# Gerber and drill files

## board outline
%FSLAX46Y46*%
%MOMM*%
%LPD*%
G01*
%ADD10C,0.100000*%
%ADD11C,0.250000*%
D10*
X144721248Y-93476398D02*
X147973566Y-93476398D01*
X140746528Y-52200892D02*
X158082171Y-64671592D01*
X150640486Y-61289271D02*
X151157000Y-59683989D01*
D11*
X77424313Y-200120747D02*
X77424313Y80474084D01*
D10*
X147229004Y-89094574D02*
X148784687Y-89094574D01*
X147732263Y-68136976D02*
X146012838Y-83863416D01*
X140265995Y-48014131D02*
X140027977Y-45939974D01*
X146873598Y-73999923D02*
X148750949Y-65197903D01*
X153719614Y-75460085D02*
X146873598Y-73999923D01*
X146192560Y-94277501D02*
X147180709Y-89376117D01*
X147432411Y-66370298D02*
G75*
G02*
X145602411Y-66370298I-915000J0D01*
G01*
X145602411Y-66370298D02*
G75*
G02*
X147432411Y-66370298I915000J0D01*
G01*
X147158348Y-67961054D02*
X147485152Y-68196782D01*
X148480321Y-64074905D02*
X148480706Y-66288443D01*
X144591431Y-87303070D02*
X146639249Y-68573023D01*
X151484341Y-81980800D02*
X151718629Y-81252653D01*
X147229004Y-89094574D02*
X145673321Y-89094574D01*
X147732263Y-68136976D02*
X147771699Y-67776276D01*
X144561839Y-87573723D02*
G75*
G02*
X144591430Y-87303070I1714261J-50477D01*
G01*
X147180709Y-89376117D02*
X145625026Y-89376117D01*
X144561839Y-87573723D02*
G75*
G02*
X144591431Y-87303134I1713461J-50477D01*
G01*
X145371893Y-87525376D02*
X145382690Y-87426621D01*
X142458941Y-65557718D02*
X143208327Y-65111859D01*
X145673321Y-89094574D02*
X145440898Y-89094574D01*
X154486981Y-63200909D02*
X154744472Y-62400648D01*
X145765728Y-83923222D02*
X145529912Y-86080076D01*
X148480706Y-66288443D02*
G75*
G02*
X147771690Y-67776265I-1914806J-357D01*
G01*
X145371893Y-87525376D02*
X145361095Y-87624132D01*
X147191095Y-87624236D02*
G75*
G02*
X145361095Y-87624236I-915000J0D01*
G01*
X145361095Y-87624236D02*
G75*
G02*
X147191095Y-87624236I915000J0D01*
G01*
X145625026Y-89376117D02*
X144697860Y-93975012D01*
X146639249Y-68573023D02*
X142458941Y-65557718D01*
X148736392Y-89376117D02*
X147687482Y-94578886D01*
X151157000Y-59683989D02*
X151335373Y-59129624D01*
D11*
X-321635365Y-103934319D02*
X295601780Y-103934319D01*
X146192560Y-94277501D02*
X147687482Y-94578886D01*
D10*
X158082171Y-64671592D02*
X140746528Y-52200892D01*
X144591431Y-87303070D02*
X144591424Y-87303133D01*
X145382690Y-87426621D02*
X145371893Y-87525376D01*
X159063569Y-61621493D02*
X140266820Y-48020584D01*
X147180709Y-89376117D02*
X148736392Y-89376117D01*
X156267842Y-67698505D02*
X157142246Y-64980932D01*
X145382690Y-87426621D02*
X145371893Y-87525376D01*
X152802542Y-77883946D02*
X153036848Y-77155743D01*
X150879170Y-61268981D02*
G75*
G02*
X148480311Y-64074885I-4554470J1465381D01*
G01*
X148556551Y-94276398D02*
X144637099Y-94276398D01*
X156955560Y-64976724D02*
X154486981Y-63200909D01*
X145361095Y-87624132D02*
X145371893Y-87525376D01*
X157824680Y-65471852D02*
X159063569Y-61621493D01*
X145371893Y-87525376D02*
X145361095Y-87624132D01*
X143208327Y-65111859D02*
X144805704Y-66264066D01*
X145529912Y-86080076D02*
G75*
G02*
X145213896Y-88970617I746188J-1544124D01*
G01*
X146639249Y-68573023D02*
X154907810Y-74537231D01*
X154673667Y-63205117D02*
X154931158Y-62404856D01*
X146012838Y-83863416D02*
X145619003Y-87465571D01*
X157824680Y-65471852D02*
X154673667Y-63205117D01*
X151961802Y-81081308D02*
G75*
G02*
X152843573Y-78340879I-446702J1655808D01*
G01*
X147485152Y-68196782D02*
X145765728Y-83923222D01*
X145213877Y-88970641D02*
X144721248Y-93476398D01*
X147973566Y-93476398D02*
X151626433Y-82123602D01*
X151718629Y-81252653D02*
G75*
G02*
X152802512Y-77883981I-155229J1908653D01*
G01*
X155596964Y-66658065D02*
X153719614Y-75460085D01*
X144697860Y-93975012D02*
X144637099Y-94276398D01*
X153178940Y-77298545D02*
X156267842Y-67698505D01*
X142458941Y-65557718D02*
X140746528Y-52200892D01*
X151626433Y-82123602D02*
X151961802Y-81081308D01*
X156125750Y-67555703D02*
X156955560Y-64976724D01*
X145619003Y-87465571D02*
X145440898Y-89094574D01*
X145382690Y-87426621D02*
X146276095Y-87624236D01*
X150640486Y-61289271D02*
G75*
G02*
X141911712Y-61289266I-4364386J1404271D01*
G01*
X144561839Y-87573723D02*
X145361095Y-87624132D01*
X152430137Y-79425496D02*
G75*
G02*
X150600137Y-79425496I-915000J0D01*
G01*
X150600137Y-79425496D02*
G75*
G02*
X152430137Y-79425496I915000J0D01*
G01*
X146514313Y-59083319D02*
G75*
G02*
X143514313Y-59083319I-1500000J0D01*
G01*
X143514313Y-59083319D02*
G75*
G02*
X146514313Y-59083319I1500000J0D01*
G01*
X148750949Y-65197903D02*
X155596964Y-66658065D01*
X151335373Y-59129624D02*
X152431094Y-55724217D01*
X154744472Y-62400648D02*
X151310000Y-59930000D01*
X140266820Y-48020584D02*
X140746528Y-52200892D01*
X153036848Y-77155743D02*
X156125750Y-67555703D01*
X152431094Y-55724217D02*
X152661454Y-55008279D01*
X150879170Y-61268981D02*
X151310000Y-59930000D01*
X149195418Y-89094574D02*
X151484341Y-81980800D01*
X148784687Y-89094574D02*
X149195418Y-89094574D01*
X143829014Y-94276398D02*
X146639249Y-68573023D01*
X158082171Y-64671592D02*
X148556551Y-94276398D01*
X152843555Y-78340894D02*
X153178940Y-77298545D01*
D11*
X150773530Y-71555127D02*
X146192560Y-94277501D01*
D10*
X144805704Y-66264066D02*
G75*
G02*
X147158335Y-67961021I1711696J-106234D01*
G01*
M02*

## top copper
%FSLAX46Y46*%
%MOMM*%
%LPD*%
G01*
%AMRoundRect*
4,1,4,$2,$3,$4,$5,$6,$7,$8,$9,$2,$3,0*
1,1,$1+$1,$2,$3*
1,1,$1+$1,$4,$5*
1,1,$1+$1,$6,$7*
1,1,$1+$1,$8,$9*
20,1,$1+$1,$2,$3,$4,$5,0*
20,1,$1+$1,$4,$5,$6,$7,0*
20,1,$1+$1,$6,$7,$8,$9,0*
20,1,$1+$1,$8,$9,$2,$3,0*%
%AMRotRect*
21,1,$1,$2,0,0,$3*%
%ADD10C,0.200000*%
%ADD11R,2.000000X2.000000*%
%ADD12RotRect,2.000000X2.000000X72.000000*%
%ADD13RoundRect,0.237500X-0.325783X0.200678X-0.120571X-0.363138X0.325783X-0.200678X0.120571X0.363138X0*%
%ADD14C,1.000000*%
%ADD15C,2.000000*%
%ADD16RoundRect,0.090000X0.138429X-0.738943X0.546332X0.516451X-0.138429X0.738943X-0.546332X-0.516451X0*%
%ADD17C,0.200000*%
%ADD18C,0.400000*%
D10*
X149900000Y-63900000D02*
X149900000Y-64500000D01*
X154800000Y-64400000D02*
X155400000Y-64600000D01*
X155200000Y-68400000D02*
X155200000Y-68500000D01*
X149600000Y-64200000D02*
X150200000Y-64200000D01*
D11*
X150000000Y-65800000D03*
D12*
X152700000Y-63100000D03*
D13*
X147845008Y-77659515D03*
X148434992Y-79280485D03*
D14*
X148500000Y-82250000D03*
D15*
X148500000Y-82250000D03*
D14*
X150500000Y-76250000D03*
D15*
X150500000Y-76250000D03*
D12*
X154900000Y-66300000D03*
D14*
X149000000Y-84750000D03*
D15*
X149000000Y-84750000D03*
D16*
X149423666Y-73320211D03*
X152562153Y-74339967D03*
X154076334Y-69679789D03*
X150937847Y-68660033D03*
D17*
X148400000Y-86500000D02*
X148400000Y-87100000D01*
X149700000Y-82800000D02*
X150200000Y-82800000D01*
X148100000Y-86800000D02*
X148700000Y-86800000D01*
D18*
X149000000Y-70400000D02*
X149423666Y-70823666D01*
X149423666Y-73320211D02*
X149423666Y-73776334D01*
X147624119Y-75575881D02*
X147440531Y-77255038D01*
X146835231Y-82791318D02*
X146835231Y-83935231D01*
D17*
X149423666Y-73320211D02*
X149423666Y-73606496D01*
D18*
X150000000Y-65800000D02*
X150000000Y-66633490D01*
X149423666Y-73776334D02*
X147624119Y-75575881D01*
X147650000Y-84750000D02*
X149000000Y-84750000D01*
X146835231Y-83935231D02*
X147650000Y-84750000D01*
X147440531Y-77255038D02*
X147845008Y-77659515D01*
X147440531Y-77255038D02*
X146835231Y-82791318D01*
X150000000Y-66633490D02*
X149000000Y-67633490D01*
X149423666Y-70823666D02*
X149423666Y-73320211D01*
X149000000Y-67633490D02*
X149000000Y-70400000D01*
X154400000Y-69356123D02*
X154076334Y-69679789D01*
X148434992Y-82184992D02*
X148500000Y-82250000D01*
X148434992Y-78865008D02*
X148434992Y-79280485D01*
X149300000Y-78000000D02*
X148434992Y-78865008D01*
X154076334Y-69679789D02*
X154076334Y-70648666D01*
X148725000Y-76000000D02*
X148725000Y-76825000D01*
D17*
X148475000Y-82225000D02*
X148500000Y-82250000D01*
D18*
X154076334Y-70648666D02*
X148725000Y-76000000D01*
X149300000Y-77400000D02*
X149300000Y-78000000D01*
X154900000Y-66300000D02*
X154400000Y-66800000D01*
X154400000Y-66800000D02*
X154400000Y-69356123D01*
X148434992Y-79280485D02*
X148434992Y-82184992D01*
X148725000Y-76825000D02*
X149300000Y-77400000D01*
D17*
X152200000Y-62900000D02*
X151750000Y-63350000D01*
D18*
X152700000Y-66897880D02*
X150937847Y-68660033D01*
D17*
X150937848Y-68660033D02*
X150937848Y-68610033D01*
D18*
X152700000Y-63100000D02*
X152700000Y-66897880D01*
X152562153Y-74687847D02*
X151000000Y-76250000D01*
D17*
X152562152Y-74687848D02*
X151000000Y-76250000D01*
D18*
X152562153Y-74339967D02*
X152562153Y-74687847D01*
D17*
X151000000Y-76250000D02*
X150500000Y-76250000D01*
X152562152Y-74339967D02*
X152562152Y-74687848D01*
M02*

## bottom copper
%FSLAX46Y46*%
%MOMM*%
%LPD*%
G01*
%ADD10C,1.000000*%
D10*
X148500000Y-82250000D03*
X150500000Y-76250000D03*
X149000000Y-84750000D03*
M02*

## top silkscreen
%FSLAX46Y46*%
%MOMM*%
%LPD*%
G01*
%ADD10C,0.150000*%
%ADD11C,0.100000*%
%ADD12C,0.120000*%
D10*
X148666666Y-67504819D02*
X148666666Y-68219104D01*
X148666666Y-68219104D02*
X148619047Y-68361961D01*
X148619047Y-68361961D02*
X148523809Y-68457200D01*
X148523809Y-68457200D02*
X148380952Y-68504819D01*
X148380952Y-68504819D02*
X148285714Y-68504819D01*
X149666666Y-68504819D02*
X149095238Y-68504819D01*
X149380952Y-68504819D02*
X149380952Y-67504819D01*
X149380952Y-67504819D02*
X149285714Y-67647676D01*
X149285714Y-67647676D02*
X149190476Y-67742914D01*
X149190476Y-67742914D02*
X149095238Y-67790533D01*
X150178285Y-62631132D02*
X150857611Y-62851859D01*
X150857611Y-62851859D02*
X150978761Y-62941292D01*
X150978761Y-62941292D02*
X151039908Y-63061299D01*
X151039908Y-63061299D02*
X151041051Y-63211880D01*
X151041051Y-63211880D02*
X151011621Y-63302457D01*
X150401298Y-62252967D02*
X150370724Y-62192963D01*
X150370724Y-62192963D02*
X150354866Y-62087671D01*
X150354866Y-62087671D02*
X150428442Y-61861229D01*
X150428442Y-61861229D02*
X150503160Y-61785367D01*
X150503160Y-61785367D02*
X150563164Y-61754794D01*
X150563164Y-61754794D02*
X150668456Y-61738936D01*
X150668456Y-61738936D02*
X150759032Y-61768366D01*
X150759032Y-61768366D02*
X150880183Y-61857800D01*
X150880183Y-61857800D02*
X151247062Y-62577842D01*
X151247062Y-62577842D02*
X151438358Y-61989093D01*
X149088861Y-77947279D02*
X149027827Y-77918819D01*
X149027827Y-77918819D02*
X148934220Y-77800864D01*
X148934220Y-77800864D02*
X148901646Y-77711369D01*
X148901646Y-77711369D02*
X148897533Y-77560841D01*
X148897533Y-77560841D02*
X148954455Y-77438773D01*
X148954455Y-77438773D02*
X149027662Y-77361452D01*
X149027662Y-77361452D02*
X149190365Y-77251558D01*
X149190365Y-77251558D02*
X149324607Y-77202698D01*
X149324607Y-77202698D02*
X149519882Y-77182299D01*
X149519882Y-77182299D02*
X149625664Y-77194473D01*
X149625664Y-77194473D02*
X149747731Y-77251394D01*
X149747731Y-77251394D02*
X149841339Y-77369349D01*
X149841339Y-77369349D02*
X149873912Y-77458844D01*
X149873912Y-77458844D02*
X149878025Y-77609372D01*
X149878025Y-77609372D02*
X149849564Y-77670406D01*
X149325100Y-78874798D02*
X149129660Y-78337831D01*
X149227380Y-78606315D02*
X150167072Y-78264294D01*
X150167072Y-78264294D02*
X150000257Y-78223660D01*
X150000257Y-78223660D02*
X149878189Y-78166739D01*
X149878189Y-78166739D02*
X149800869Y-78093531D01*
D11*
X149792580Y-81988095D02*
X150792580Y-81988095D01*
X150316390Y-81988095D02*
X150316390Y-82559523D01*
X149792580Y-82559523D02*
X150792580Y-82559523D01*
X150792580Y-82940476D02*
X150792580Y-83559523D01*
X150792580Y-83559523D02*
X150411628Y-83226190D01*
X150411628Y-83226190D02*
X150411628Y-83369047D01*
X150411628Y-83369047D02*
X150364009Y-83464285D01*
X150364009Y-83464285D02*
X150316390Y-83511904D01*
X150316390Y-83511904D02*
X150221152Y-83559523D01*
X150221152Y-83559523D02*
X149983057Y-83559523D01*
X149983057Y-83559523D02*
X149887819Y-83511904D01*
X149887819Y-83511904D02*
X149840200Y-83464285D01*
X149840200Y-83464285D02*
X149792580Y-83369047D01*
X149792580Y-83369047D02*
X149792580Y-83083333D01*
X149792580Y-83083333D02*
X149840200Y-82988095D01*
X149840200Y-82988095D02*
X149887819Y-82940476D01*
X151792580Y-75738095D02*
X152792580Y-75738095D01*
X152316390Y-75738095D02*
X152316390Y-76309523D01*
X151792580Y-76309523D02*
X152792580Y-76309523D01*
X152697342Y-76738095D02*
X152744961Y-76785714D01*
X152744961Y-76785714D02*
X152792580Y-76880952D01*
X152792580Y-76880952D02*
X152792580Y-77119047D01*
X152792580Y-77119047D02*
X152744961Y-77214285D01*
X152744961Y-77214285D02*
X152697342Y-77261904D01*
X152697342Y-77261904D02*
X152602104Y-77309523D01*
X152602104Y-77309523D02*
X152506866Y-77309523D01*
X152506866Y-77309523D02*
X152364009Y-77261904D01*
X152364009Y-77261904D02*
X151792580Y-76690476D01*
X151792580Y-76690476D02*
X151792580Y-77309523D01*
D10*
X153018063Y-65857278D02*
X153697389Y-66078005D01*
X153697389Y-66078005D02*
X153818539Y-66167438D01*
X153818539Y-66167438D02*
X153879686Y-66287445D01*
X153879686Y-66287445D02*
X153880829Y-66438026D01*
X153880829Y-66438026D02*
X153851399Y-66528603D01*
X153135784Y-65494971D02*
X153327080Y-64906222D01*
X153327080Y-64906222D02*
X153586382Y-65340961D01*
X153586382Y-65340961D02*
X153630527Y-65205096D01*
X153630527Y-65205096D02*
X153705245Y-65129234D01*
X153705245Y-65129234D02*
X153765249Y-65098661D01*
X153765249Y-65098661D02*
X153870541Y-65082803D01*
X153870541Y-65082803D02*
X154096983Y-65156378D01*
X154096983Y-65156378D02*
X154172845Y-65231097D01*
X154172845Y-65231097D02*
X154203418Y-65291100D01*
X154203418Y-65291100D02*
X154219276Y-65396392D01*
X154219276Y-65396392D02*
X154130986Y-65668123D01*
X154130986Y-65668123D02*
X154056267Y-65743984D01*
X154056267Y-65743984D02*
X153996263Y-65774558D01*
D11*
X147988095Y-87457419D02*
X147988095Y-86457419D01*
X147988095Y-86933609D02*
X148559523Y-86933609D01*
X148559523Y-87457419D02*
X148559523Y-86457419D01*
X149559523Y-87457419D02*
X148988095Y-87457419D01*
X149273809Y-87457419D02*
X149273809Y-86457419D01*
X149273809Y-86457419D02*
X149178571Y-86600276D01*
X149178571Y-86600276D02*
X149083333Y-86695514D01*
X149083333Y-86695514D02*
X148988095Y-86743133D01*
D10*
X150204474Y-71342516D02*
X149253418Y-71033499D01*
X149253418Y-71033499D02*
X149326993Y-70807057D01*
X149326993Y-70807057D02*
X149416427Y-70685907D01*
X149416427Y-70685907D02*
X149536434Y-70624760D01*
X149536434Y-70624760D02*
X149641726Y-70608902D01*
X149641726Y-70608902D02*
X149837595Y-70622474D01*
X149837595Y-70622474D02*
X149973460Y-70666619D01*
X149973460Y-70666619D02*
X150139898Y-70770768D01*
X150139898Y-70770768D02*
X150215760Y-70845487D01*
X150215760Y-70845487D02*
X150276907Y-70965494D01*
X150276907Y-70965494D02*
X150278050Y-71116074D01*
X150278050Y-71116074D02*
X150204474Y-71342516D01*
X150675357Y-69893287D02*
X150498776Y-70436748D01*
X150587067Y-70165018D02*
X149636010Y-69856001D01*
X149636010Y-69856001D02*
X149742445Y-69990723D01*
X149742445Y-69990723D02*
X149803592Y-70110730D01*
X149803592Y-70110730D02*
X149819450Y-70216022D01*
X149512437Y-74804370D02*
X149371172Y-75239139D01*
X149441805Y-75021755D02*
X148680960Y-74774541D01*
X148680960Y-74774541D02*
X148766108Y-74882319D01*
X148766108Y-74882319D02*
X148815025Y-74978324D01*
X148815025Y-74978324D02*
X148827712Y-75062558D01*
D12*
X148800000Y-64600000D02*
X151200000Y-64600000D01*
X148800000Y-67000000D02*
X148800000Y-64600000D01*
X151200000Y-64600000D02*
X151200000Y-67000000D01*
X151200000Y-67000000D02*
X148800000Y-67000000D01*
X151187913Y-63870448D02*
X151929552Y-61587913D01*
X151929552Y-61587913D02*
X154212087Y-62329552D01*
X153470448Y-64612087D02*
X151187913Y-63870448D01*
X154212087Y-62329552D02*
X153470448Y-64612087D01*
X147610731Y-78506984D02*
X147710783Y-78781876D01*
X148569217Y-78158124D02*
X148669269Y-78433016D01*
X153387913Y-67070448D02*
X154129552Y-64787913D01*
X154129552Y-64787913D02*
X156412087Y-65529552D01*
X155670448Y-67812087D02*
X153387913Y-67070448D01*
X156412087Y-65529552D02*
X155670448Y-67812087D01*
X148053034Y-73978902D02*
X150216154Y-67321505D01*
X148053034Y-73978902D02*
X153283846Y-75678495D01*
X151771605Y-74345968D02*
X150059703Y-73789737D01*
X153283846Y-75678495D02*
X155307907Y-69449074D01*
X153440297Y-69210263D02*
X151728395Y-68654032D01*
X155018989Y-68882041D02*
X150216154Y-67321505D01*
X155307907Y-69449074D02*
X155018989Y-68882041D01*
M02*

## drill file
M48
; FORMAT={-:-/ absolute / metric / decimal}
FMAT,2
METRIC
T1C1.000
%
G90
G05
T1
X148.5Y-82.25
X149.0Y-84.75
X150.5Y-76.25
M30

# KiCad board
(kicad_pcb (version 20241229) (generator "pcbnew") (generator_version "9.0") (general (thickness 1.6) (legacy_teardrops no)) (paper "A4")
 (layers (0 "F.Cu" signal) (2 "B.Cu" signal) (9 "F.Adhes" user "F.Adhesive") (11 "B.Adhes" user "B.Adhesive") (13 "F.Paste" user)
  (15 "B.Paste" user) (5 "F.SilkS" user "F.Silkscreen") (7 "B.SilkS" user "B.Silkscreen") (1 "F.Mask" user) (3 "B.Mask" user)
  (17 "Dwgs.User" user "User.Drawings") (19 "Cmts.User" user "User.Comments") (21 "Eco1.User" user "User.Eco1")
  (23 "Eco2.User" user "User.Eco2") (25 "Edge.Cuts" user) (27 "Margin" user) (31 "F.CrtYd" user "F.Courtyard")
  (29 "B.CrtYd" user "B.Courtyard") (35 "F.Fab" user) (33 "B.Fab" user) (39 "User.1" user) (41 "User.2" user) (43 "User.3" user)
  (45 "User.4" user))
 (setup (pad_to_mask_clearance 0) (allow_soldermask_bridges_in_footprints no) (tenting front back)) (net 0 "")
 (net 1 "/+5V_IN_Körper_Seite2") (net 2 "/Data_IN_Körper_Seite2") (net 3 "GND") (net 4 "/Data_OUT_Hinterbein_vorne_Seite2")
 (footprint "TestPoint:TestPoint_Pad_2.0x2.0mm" (layer "F.Cu") (at 150 65.8)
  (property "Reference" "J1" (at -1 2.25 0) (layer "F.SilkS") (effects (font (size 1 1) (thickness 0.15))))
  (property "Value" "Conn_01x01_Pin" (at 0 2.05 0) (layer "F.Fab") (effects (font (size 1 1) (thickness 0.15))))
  (fp_line (start -1.2 -1.2) (end 1.2 -1.2) (stroke (width 0.12) (type solid)) (layer "F.SilkS"))
  (fp_line (start -1.2 1.2) (end -1.2 -1.2) (stroke (width 0.12) (type solid)) (layer "F.SilkS"))
  (fp_line (start 1.2 -1.2) (end 1.2 1.2) (stroke (width 0.12) (type solid)) (layer "F.SilkS"))
  (fp_line (start 1.2 1.2) (end -1.2 1.2) (stroke (width 0.12) (type solid)) (layer "F.SilkS"))
  (pad "1" smd rect (at 0 0) (size 2 2) (layers "F.Cu" "F.Mask") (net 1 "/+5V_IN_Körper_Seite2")))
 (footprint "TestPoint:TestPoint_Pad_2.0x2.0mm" (layer "F.Cu") (at 152.7 63.1 72)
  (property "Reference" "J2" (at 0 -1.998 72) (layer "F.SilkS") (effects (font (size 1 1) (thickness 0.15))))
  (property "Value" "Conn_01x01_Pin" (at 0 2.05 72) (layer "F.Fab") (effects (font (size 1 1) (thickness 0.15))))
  (fp_line (start -1.2 -1.199999) (end 1.199999 -1.2) (stroke (width 0.12) (type solid)) (layer "F.SilkS"))
  (fp_line (start 1.199999 -1.2) (end 1.2 1.199999) (stroke (width 0.12) (type solid)) (layer "F.SilkS"))
  (fp_line (start -1.199999 1.2) (end -1.2 -1.199999) (stroke (width 0.12) (type solid)) (layer "F.SilkS"))
  (fp_line (start 1.2 1.199999) (end -1.199999 1.2) (stroke (width 0.12) (type solid)) (layer "F.SilkS"))
  (pad "1" smd rect (at 0 0 72) (size 2 2) (layers "F.Cu" "F.Mask") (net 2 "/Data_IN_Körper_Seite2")))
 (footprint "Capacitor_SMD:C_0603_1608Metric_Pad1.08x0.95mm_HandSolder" (layer "F.Cu") (at 148.14 78.47 -70)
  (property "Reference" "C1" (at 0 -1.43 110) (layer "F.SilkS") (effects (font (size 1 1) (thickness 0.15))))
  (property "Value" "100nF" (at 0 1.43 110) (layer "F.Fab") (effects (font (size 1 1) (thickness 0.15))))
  (fp_line (start -0.146267 0.509999) (end 0.146267 0.51) (stroke (width 0.12) (type solid)) (layer "F.SilkS"))
  (fp_line (start -0.146267 -0.51) (end 0.146267 -0.509999) (stroke (width 0.12) (type solid)) (layer "F.SilkS"))
  (pad "1" smd roundrect (at -0.8625 0 290) (size 1.075 0.95) (layers "F.Cu" "F.Mask" "F.Paste") (roundrect_rratio 0.25)
   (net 1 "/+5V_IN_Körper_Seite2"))
  (pad "2" smd roundrect (at 0.8625 0 290) (size 1.075 0.95) (layers "F.Cu" "F.Mask" "F.Paste") (roundrect_rratio 0.25) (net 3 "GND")))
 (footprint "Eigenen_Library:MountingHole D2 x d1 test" (layer "F.Cu") (at 148.5 82.25)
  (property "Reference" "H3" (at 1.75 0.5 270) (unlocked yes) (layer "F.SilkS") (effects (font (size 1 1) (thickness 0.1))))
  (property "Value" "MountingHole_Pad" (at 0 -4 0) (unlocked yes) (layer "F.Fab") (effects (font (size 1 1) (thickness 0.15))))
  (pad "1" thru_hole circle (at 0 0) (size 1 1) (drill 1) (layers "*.Cu" "*.Mask") (remove_unused_layers no) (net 3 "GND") (zone_connect 2))
  (pad "1" connect circle (at 0 0) (size 2 2) (layers "F.Cu" "F.Mask") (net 3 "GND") (zone_connect 2)))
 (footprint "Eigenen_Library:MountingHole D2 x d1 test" (layer "F.Cu") (at 150.5 76.25)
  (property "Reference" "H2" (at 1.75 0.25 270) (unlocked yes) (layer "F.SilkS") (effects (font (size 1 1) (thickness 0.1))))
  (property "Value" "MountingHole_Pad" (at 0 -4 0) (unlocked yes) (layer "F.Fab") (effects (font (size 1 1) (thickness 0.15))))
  (pad "1" thru_hole circle (at 0 0) (size 1 1) (drill 1) (layers "*.Cu" "*.Mask") (remove_unused_layers no)
   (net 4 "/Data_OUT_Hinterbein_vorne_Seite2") (zone_connect 2))
  (pad "1" connect circle (at 0 0) (size 2 2) (layers "F.Cu" "F.Mask") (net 4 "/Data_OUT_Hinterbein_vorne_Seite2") (zone_connect 2)))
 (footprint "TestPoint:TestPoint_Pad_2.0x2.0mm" (layer "F.Cu") (at 154.9 66.3 72)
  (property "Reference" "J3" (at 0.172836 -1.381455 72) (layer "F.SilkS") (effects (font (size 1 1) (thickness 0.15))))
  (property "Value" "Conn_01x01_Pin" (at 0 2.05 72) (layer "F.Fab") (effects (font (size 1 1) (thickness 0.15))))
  (fp_line (start -1.2 -1.199999) (end 1.199999 -1.2) (stroke (width 0.12) (type solid)) (layer "F.SilkS"))
  (fp_line (start 1.199999 -1.2) (end 1.2 1.199999) (stroke (width 0.12) (type solid)) (layer "F.SilkS"))
  (fp_line (start -1.199999 1.2) (end -1.2 -1.199999) (stroke (width 0.12) (type solid)) (layer "F.SilkS"))
  (fp_line (start 1.2 1.199999) (end -1.199999 1.2) (stroke (width 0.12) (type solid)) (layer "F.SilkS"))
  (pad "1" smd rect (at 0 0 72) (size 2 2) (layers "F.Cu" "F.Mask") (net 3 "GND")))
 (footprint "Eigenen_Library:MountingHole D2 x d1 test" (layer "F.Cu") (at 149 84.75)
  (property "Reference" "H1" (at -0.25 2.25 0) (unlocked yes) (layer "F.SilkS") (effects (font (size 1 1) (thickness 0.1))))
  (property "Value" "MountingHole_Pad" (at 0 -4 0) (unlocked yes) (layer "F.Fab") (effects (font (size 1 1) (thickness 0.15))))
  (pad "1" thru_hole circle (at 0 0) (size 1 1) (drill 1) (layers "*.Cu" "*.Mask") (remove_unused_layers no) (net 1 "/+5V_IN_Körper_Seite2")
   (zone_connect 2))
  (pad "1" connect circle (at 0 0) (size 2 2) (layers "F.Cu" "F.Mask") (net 1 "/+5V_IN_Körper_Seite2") (zone_connect 2)))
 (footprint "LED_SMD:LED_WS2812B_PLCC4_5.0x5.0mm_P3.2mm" (layer "F.Cu") (at 151.75 71.5 72)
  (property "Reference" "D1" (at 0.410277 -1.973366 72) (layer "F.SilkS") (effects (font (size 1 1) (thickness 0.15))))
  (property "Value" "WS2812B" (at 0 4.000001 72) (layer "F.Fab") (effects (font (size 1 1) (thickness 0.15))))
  (fp_line (start -3.500001 -2.750001) (end 3.5 -2.75) (stroke (width 0.12) (type solid)) (layer "F.SilkS"))
  (fp_line (start -3.500001 -2.750001) (end -3.5 2.75) (stroke (width 0.12) (type default)) (layer "F.SilkS"))
  (fp_line (start -2.7 0.9) (end -2.7 -0.9) (stroke (width 0.12) (type default)) (layer "F.SilkS"))
  (fp_line (start -3.5 2.75) (end 3.05 2.75) (stroke (width 0.12) (type solid)) (layer "F.SilkS"))
  (fp_line (start 2.7 0.9) (end 2.7 -0.9) (stroke (width 0.12) (type default)) (layer "F.SilkS"))
  (fp_line (start 3.5 2.299999) (end 3.5 -2.75) (stroke (width 0.12) (type default)) (layer "F.SilkS"))
  (fp_line (start 3.05 2.75) (end 3.5 2.299999) (stroke (width 0.12) (type default)) (layer "F.SilkS"))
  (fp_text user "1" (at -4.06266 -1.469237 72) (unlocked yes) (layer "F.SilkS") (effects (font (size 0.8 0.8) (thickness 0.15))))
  (pad "1" smd roundrect (at -2.45 -1.649999 72) (size 1.5 0.9) (layers "F.Cu" "F.Mask" "F.Paste") (roundrect_rratio 0.1)
   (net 1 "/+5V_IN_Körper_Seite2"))
  (pad "2" smd roundrect (at -2.45 1.650001 72) (size 1.5 0.9) (layers "F.Cu" "F.Mask" "F.Paste") (roundrect_rratio 0.1)
   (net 4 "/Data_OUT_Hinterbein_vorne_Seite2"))
  (pad "3" smd roundrect (at 2.45 1.649999 72) (size 1.5 0.9) (layers "F.Cu" "F.Mask" "F.Paste") (roundrect_rratio 0.1) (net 3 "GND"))
  (pad "4" smd roundrect (at 2.45 -1.650001 72) (size 1.5 0.9) (layers "F.Cu" "F.Mask" "F.Paste") (roundrect_rratio 0.1)
   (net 2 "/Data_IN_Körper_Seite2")))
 (gr_line (start 149.9 63.9) (end 149.9 64.5) (stroke (width 0.2) (type default)) (layer "F.Cu"))
 (gr_line (start 154.8 64.4) (end 155.4 64.6) (stroke (width 0.2) (type default)) (layer "F.Cu"))
 (gr_line (start 155.2 68.4) (end 155.2 68.5) (stroke (width 0.2) (type default)) (layer "F.Cu"))
 (gr_line (start 149.6 64.2) (end 150.2 64.2) (stroke (width 0.2) (type default)) (layer "F.Cu"))
 (gr_line (start 144.721248 93.476398) (end 147.973566 93.476398) (stroke (width 0.1) (type default)) (layer "Edge.Cuts"))
 (gr_line (start 140.746528 52.200892) (end 158.082171 64.671592) (stroke (width 0.1) (type default)) (layer "Edge.Cuts"))
 (gr_line (start 150.640486 61.289271) (end 151.157 59.683989) (stroke (width 0.1) (type default)) (layer "Edge.Cuts"))
 (gr_line (start 77.424313 200.120747) (end 77.424313 -80.474084) (stroke (width 0.25) (type default)) (layer "Edge.Cuts"))
 (gr_line (start 147.229004 89.094574) (end 148.784687 89.094574) (stroke (width 0.1) (type default)) (locked yes) (layer "Edge.Cuts"))
 (gr_line (start 147.732263 68.136976) (end 146.012838 83.863416) (stroke (width 0.1) (type default)) (locked yes) (layer "Edge.Cuts"))
 (gr_line (start 140.265995 48.014131) (end 140.027977 45.939974) (stroke (width 0.1) (type default)) (layer "Edge.Cuts"))
 (gr_line (start 146.873598 73.999923) (end 148.750949 65.197903) (stroke (width 0.1) (type default)) (layer "Edge.Cuts"))
 (gr_line (start 153.719614 75.460085) (end 146.873598 73.999923) (stroke (width 0.1) (type default)) (layer "Edge.Cuts"))
 (gr_line (start 146.19256 94.277501) (end 147.180709 89.376117) (stroke (width 0.1) (type default)) (layer "Edge.Cuts"))
 (gr_circle (center 146.517411 66.370298) (end 147.432411 66.370298) (stroke (width 0.1) (type default)) (fill no) (layer "Edge.Cuts"))
 (gr_line (start 147.158348 67.961054) (end 147.485152 68.196782) (stroke (width 0.1) (type default)) (layer "Edge.Cuts"))
 (gr_line (start 148.480321 64.074905) (end 148.480706 66.288443) (stroke (width 0.1) (type default)) (locked yes) (layer "Edge.Cuts"))
 (gr_line (start 144.591431 87.30307) (end 146.639249 68.573023) (stroke (width 0.1) (type default)) (layer "Edge.Cuts"))
 (gr_line (start 151.484341 81.9808) (end 151.718629 81.252653) (stroke (width 0.1) (type default)) (locked yes) (layer "Edge.Cuts"))
 (gr_line (start 147.229004 89.094574) (end 145.673321 89.094574) (stroke (width 0.1) (type default)) (locked yes) (layer "Edge.Cuts"))
 (gr_line (start 147.732263 68.136976) (end 147.771699 67.776276) (stroke (width 0.1) (type default)) (locked yes) (layer "Edge.Cuts"))
 (gr_arc (start 144.561839 87.573723) (mid 144.571252 87.43784) (end 144.591431 87.30307) (stroke (width 0.1) (type default))
  (layer "Edge.Cuts"))
 (gr_line (start 147.180709 89.376117) (end 145.625026 89.376117) (stroke (width 0.1) (type default)) (layer "Edge.Cuts"))
 (gr_arc (start 144.561839 87.573723) (mid 144.571252 87.43784) (end 144.591424 87.303133) (stroke (width 0.1) (type default))
  (layer "Edge.Cuts"))
 (gr_line (start 145.371893 87.525376) (end 145.38269 87.426621) (stroke (width 0.1) (type default)) (layer "Edge.Cuts"))
 (gr_line (start 142.458941 65.557718) (end 143.208327 65.111859) (stroke (width 0.1) (type default)) (layer "Edge.Cuts"))
 (gr_line (start 145.673321 89.094574) (end 145.440898 89.094574) (stroke (width 0.1) (type default)) (locked yes) (layer "Edge.Cuts"))
 (gr_line (start 154.486981 63.200909) (end 154.744472 62.400648) (stroke (width 0.1) (type default)) (locked yes) (layer "Edge.Cuts"))
 (gr_line (start 145.765728 83.923222) (end 145.529912 86.080076) (stroke (width 0.1) (type default)) (layer "Edge.Cuts"))
 (gr_arc (start 148.480706 66.288443) (mid 148.294469 67.112549) (end 147.771699 67.776276) (stroke (width 0.1) (type default)) (locked yes)
  (layer "Edge.Cuts"))
 (gr_line (start 145.371893 87.525376) (end 145.361095 87.624132) (stroke (width 0.1) (type default)) (layer "Edge.Cuts"))
 (gr_circle (center 146.276095 87.624236) (end 147.191095 87.624236) (stroke (width 0.1) (type default)) (fill no) (layer "Edge.Cuts"))
 (gr_line (start 145.625026 89.376117) (end 144.69786 93.975012) (stroke (width 0.1) (type default)) (layer "Edge.Cuts"))
 (gr_line (start 146.639249 68.573023) (end 142.458941 65.557718) (stroke (width 0.1) (type default)) (layer "Edge.Cuts"))
 (gr_line (start 148.736392 89.376117) (end 147.687482 94.578886) (stroke (width 0.1) (type default)) (layer "Edge.Cuts"))
 (gr_line (start 151.157 59.683989) (end 151.335373 59.129624) (stroke (width 0.1) (type default)) (layer "Edge.Cuts"))
 (gr_line (start -321.635365 103.934319) (end 295.60178 103.934319) (stroke (width 0.25) (type default)) (layer "Edge.Cuts"))
 (gr_line (start 146.19256 94.277501) (end 147.687482 94.578886) (stroke (width 0.25) (type default)) (layer "Edge.Cuts"))
 (gr_line (start 158.082171 64.671592) (end 140.746528 52.200892) (stroke (width 0.1) (type default)) (layer "Edge.Cuts"))
 (gr_line (start 144.591431 87.30307) (end 144.591424 87.303133) (stroke (width 0.1) (type default)) (layer "Edge.Cuts"))
 (gr_line (start 145.38269 87.426621) (end 145.371893 87.525376) (stroke (width 0.1) (type default)) (layer "Edge.Cuts"))
 (gr_line (start 159.063569 61.621493) (end 140.26682 48.020584) (stroke (width 0.1) (type default)) (layer "Edge.Cuts"))
 (gr_line (start 147.180709 89.376117) (end 148.736392 89.376117) (stroke (width 0.1) (type default)) (layer "Edge.Cuts"))
 (gr_line (start 156.267842 67.698505) (end 157.142246 64.980932) (stroke (width 0.1) (type default)) (layer "Edge.Cuts"))
 (gr_line (start 145.38269 87.426621) (end 145.371893 87.525376) (stroke (width 0.1) (type default)) (layer "Edge.Cuts"))
 (gr_line (start 152.802542 77.883946) (end 153.036848 77.155743) (stroke (width 0.1) (type default)) (locked yes) (layer "Edge.Cuts"))
 (gr_arc (start 150.87917 61.268981) (mid 149.961258 62.912638) (end 148.480321 64.074905) (stroke (width 0.1) (type default)) (locked yes)
  (layer "Edge.Cuts"))
 (gr_line (start 148.556551 94.276398) (end 144.637099 94.276398) (stroke (width 0.1) (type default)) (layer "Edge.Cuts"))
 (gr_line (start 156.95556 64.976724) (end 154.486981 63.200909) (stroke (width 0.1) (type default)) (locked yes) (layer "Edge.Cuts"))
 (gr_line (start 145.361095 87.624132) (end 145.371893 87.525376) (stroke (width 0.1) (type default)) (layer "Edge.Cuts"))
 (gr_line (start 157.82468 65.471852) (end 159.063569 61.621493) (stroke (width 0.1) (type default)) (layer "Edge.Cuts"))
 (gr_line (start 145.371893 87.525376) (end 145.361095 87.624132) (stroke (width 0.1) (type default)) (layer "Edge.Cuts"))
 (gr_line (start 143.208327 65.111859) (end 144.805704 66.264066) (stroke (width 0.1) (type default)) (layer "Edge.Cuts"))
 (gr_arc (start 145.529912 86.080076) (mid 147.980947 87.810604) (end 145.213877 88.970641) (stroke (width 0.1) (type default))
  (layer "Edge.Cuts"))
 (gr_line (start 146.639249 68.573023) (end 154.90781 74.537231) (stroke (width 0.1) (type default)) (layer "Edge.Cuts"))
 (gr_line (start 154.673667 63.205117) (end 154.931158 62.404856) (stroke (width 0.1) (type default)) (layer "Edge.Cuts"))
 (gr_line (start 146.012838 83.863416) (end 145.619003 87.465571) (stroke (width 0.1) (type default)) (locked yes) (layer "Edge.Cuts"))
 (gr_line (start 157.82468 65.471852) (end 154.673667 63.205117) (stroke (width 0.1) (type default)) (layer "Edge.Cuts"))
 (gr_arc (start 151.961802 81.081308) (mid 149.882552 78.900244) (end 152.843555 78.340894) (stroke (width 0.1) (type default))
  (layer "Edge.Cuts"))
 (gr_line (start 147.485152 68.196782) (end 145.765728 83.923222) (stroke (width 0.1) (type default)) (layer "Edge.Cuts"))
 (gr_line (start 145.213877 88.970641) (end 144.721248 93.476398) (stroke (width 0.1) (type default)) (layer "Edge.Cuts"))
 (gr_line (start 147.973566 93.476398) (end 151.626433 82.123602) (stroke (width 0.1) (type default)) (layer "Edge.Cuts"))
 (gr_arc (start 151.718629 81.252653) (mid 149.740465 78.757439) (end 152.802542 77.883946) (stroke (width 0.1) (type default)) (locked yes)
  (layer "Edge.Cuts"))
 (gr_line (start 155.596964 66.658065) (end 153.719614 75.460085) (stroke (width 0.1) (type default)) (layer "Edge.Cuts"))
 (gr_line (start 144.69786 93.975012) (end 144.637099 94.276398) (stroke (width 0.1) (type default)) (layer "Edge.Cuts"))
 (gr_line (start 153.17894 77.298545) (end 156.267842 67.698505) (stroke (width 0.1) (type default)) (layer "Edge.Cuts"))
 (gr_line (start 142.458941 65.557718) (end 140.746528 52.200892) (stroke (width 0.1) (type default)) (layer "Edge.Cuts"))
 (gr_line (start 151.626433 82.123602) (end 151.961802 81.081308) (stroke (width 0.1) (type default)) (layer "Edge.Cuts"))
 (gr_line (start 156.12575 67.555703) (end 156.95556 64.976724) (stroke (width 0.1) (type default)) (locked yes) (layer "Edge.Cuts"))
 (gr_line (start 145.619003 87.465571) (end 145.440898 89.094574) (stroke (width 0.1) (type default)) (locked yes) (layer "Edge.Cuts"))
 (gr_line (start 145.38269 87.426621) (end 146.276095 87.624236) (stroke (width 0.1) (type default)) (layer "Edge.Cuts"))
 (gr_arc (start 150.640486 61.289271) (mid 146.276096 64.469735) (end 141.911704 61.289269) (stroke (width 0.1) (type default))
  (layer "Edge.Cuts"))
 (gr_line (start 144.561839 87.573723) (end 145.361095 87.624132) (stroke (width 0.1) (type default)) (layer "Edge.Cuts"))
 (gr_circle (center 151.515137 79.425496) (end 152.430137 79.425496) (stroke (width 0.1) (type default)) (fill no) (layer "Edge.Cuts"))
 (gr_circle (center 145.014313 59.083319) (end 146.514313 59.083319) (stroke (width 0.1) (type default)) (fill no) (layer "Edge.Cuts"))
 (gr_line (start 148.750949 65.197903) (end 155.596964 66.658065) (stroke (width 0.1) (type default)) (layer "Edge.Cuts"))
 (gr_line (start 151.335373 59.129624) (end 152.431094 55.724217) (stroke (width 0.1) (type default)) (layer "Edge.Cuts"))
 (gr_line (start 154.744472 62.400648) (end 151.31 59.93) (stroke (width 0.1) (type default)) (locked yes) (layer "Edge.Cuts"))
 (gr_line (start 140.26682 48.020584) (end 140.746528 52.200892) (stroke (width 0.1) (type default)) (layer "Edge.Cuts"))
 (gr_line (start 153.036848 77.155743) (end 156.12575 67.555703) (stroke (width 0.1) (type default)) (locked yes) (layer "Edge.Cuts"))
 (gr_line (start 152.431094 55.724217) (end 152.661454 55.008279) (stroke (width 0.1) (type default)) (layer "Edge.Cuts"))
 (gr_line (start 150.87917 61.268981) (end 151.31 59.93) (stroke (width 0.1) (type default)) (locked yes) (layer "Edge.Cuts"))
 (gr_line (start 149.195418 89.094574) (end 151.484341 81.9808) (stroke (width 0.1) (type default)) (locked yes) (layer "Edge.Cuts"))
 (gr_line (start 148.784687 89.094574) (end 149.195418 89.094574) (stroke (width 0.1) (type default)) (locked yes) (layer "Edge.Cuts"))
 (gr_line (start 143.829014 94.276398) (end 146.639249 68.573023) (stroke (width 0.1) (type default)) (layer "Edge.Cuts"))
 (gr_line (start 158.082171 64.671592) (end 148.556551 94.276398) (stroke (width 0.1) (type default)) (layer "Edge.Cuts"))
 (gr_line (start 152.843555 78.340894) (end 153.17894 77.298545) (stroke (width 0.1) (type default)) (layer "Edge.Cuts"))
 (gr_line (start 150.77353 71.555127) (end 146.19256 94.277501) (stroke (width 0.25) (type default)) (layer "Edge.Cuts"))
 (gr_arc (start 144.805704 66.264066) (mid 147.520699 64.979382) (end 147.158348 67.961054) (stroke (width 0.1) (type default))
  (layer "Edge.Cuts"))
 (segment (start 148.4 86.5) (end 148.4 87.1) (width 0.2) (layer "F.Cu") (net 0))
 (segment (start 149.7 82.8) (end 150.2 82.8) (width 0.2) (layer "F.Cu") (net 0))
 (segment (start 148.1 86.8) (end 148.7 86.8) (width 0.2) (layer "F.Cu") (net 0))
 (segment (start 149 70.4) (end 149.423666 70.823666) (width 0.4) (layer "F.Cu") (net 1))
 (segment (start 149.423666 73.320211) (end 149.423666 73.776334) (width 0.4) (layer "F.Cu") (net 1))
 (segment (start 147.624119 75.575881) (end 147.440531 77.255038) (width 0.4) (layer "F.Cu") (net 1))
 (segment (start 146.835231 82.791318) (end 146.835231 83.935231) (width 0.4) (layer "F.Cu") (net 1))
 (segment (start 149.423666 73.320211) (end 149.423666 73.606496) (width 0.2) (layer "F.Cu") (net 1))
 (segment (start 150 65.8) (end 150 66.63349) (width 0.4) (layer "F.Cu") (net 1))
 (segment (start 149.423666 73.776334) (end 147.624119 75.575881) (width 0.4) (layer "F.Cu") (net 1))
 (segment (start 147.65 84.75) (end 149 84.75) (width 0.4) (layer "F.Cu") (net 1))
 (segment (start 146.835231 83.935231) (end 147.65 84.75) (width 0.4) (layer "F.Cu") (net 1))
 (segment (start 147.440531 77.255038) (end 147.845008 77.659515) (width 0.4) (layer "F.Cu") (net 1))
 (segment (start 147.440531 77.255038) (end 146.835231 82.791318) (width 0.4) (layer "F.Cu") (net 1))
 (segment (start 150 66.63349) (end 149 67.63349) (width 0.4) (layer "F.Cu") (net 1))
 (segment (start 149.423666 70.823666) (end 149.423666 73.320211) (width 0.4) (layer "F.Cu") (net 1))
 (segment (start 149 67.63349) (end 149 70.4) (width 0.4) (layer "F.Cu") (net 1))
 (segment (start 154.4 69.356123) (end 154.076334 69.679789) (width 0.4) (layer "F.Cu") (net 3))
 (segment (start 148.434992 82.184992) (end 148.5 82.25) (width 0.4) (layer "F.Cu") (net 3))
 (segment (start 148.434992 78.865008) (end 148.434992 79.280485) (width 0.4) (layer "F.Cu") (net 3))
 (segment (start 149.3 78) (end 148.434992 78.865008) (width 0.4) (layer "F.Cu") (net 3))
 (segment (start 154.076334 69.679789) (end 154.076334 70.648666) (width 0.4) (layer "F.Cu") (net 3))
 (segment (start 148.725 76) (end 148.725 76.825) (width 0.4) (layer "F.Cu") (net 3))
 (segment (start 148.475 82.225) (end 148.5 82.25) (width 0.2) (layer "F.Cu") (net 3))
 (segment (start 154.076334 70.648666) (end 148.725 76) (width 0.4) (layer "F.Cu") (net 3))
 (segment (start 149.3 77.4) (end 149.3 78) (width 0.4) (layer "F.Cu") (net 3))
 (segment (start 154.9 66.3) (end 154.4 66.8) (width 0.4) (layer "F.Cu") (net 3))
 (segment (start 154.4 66.8) (end 154.4 69.356123) (width 0.4) (layer "F.Cu") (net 3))
 (segment (start 148.434992 79.280485) (end 148.434992 82.184992) (width 0.4) (layer "F.Cu") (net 3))
 (segment (start 148.725 76.825) (end 149.3 77.4) (width 0.4) (layer "F.Cu") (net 3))
 (segment (start 152.2 62.9) (end 151.75 63.35) (width 0.2) (layer "F.Cu") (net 2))
 (segment (start 152.7 66.89788) (end 150.937847 68.660033) (width 0.4) (layer "F.Cu") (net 2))
 (segment (start 150.937848 68.660033) (end 150.937848 68.610033) (width 0.2) (layer "F.Cu") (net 2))
 (segment (start 152.7 63.1) (end 152.7 66.89788) (width 0.4) (layer "F.Cu") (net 2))
 (segment (start 152.562153 74.687847) (end 151 76.25) (width 0.4) (layer "F.Cu") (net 4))
 (segment (start 152.562152 74.687848) (end 151 76.25) (width 0.2) (layer "F.Cu") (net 4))
 (segment (start 152.562153 74.339967) (end 152.562153 74.687847) (width 0.4) (layer "F.Cu") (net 4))
 (segment (start 151 76.25) (end 150.5 76.25) (width 0.2) (layer "F.Cu") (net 4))
 (segment (start 152.562152 74.339967) (end 152.562152 74.687848) (width 0.2) (layer "F.Cu") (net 4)))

